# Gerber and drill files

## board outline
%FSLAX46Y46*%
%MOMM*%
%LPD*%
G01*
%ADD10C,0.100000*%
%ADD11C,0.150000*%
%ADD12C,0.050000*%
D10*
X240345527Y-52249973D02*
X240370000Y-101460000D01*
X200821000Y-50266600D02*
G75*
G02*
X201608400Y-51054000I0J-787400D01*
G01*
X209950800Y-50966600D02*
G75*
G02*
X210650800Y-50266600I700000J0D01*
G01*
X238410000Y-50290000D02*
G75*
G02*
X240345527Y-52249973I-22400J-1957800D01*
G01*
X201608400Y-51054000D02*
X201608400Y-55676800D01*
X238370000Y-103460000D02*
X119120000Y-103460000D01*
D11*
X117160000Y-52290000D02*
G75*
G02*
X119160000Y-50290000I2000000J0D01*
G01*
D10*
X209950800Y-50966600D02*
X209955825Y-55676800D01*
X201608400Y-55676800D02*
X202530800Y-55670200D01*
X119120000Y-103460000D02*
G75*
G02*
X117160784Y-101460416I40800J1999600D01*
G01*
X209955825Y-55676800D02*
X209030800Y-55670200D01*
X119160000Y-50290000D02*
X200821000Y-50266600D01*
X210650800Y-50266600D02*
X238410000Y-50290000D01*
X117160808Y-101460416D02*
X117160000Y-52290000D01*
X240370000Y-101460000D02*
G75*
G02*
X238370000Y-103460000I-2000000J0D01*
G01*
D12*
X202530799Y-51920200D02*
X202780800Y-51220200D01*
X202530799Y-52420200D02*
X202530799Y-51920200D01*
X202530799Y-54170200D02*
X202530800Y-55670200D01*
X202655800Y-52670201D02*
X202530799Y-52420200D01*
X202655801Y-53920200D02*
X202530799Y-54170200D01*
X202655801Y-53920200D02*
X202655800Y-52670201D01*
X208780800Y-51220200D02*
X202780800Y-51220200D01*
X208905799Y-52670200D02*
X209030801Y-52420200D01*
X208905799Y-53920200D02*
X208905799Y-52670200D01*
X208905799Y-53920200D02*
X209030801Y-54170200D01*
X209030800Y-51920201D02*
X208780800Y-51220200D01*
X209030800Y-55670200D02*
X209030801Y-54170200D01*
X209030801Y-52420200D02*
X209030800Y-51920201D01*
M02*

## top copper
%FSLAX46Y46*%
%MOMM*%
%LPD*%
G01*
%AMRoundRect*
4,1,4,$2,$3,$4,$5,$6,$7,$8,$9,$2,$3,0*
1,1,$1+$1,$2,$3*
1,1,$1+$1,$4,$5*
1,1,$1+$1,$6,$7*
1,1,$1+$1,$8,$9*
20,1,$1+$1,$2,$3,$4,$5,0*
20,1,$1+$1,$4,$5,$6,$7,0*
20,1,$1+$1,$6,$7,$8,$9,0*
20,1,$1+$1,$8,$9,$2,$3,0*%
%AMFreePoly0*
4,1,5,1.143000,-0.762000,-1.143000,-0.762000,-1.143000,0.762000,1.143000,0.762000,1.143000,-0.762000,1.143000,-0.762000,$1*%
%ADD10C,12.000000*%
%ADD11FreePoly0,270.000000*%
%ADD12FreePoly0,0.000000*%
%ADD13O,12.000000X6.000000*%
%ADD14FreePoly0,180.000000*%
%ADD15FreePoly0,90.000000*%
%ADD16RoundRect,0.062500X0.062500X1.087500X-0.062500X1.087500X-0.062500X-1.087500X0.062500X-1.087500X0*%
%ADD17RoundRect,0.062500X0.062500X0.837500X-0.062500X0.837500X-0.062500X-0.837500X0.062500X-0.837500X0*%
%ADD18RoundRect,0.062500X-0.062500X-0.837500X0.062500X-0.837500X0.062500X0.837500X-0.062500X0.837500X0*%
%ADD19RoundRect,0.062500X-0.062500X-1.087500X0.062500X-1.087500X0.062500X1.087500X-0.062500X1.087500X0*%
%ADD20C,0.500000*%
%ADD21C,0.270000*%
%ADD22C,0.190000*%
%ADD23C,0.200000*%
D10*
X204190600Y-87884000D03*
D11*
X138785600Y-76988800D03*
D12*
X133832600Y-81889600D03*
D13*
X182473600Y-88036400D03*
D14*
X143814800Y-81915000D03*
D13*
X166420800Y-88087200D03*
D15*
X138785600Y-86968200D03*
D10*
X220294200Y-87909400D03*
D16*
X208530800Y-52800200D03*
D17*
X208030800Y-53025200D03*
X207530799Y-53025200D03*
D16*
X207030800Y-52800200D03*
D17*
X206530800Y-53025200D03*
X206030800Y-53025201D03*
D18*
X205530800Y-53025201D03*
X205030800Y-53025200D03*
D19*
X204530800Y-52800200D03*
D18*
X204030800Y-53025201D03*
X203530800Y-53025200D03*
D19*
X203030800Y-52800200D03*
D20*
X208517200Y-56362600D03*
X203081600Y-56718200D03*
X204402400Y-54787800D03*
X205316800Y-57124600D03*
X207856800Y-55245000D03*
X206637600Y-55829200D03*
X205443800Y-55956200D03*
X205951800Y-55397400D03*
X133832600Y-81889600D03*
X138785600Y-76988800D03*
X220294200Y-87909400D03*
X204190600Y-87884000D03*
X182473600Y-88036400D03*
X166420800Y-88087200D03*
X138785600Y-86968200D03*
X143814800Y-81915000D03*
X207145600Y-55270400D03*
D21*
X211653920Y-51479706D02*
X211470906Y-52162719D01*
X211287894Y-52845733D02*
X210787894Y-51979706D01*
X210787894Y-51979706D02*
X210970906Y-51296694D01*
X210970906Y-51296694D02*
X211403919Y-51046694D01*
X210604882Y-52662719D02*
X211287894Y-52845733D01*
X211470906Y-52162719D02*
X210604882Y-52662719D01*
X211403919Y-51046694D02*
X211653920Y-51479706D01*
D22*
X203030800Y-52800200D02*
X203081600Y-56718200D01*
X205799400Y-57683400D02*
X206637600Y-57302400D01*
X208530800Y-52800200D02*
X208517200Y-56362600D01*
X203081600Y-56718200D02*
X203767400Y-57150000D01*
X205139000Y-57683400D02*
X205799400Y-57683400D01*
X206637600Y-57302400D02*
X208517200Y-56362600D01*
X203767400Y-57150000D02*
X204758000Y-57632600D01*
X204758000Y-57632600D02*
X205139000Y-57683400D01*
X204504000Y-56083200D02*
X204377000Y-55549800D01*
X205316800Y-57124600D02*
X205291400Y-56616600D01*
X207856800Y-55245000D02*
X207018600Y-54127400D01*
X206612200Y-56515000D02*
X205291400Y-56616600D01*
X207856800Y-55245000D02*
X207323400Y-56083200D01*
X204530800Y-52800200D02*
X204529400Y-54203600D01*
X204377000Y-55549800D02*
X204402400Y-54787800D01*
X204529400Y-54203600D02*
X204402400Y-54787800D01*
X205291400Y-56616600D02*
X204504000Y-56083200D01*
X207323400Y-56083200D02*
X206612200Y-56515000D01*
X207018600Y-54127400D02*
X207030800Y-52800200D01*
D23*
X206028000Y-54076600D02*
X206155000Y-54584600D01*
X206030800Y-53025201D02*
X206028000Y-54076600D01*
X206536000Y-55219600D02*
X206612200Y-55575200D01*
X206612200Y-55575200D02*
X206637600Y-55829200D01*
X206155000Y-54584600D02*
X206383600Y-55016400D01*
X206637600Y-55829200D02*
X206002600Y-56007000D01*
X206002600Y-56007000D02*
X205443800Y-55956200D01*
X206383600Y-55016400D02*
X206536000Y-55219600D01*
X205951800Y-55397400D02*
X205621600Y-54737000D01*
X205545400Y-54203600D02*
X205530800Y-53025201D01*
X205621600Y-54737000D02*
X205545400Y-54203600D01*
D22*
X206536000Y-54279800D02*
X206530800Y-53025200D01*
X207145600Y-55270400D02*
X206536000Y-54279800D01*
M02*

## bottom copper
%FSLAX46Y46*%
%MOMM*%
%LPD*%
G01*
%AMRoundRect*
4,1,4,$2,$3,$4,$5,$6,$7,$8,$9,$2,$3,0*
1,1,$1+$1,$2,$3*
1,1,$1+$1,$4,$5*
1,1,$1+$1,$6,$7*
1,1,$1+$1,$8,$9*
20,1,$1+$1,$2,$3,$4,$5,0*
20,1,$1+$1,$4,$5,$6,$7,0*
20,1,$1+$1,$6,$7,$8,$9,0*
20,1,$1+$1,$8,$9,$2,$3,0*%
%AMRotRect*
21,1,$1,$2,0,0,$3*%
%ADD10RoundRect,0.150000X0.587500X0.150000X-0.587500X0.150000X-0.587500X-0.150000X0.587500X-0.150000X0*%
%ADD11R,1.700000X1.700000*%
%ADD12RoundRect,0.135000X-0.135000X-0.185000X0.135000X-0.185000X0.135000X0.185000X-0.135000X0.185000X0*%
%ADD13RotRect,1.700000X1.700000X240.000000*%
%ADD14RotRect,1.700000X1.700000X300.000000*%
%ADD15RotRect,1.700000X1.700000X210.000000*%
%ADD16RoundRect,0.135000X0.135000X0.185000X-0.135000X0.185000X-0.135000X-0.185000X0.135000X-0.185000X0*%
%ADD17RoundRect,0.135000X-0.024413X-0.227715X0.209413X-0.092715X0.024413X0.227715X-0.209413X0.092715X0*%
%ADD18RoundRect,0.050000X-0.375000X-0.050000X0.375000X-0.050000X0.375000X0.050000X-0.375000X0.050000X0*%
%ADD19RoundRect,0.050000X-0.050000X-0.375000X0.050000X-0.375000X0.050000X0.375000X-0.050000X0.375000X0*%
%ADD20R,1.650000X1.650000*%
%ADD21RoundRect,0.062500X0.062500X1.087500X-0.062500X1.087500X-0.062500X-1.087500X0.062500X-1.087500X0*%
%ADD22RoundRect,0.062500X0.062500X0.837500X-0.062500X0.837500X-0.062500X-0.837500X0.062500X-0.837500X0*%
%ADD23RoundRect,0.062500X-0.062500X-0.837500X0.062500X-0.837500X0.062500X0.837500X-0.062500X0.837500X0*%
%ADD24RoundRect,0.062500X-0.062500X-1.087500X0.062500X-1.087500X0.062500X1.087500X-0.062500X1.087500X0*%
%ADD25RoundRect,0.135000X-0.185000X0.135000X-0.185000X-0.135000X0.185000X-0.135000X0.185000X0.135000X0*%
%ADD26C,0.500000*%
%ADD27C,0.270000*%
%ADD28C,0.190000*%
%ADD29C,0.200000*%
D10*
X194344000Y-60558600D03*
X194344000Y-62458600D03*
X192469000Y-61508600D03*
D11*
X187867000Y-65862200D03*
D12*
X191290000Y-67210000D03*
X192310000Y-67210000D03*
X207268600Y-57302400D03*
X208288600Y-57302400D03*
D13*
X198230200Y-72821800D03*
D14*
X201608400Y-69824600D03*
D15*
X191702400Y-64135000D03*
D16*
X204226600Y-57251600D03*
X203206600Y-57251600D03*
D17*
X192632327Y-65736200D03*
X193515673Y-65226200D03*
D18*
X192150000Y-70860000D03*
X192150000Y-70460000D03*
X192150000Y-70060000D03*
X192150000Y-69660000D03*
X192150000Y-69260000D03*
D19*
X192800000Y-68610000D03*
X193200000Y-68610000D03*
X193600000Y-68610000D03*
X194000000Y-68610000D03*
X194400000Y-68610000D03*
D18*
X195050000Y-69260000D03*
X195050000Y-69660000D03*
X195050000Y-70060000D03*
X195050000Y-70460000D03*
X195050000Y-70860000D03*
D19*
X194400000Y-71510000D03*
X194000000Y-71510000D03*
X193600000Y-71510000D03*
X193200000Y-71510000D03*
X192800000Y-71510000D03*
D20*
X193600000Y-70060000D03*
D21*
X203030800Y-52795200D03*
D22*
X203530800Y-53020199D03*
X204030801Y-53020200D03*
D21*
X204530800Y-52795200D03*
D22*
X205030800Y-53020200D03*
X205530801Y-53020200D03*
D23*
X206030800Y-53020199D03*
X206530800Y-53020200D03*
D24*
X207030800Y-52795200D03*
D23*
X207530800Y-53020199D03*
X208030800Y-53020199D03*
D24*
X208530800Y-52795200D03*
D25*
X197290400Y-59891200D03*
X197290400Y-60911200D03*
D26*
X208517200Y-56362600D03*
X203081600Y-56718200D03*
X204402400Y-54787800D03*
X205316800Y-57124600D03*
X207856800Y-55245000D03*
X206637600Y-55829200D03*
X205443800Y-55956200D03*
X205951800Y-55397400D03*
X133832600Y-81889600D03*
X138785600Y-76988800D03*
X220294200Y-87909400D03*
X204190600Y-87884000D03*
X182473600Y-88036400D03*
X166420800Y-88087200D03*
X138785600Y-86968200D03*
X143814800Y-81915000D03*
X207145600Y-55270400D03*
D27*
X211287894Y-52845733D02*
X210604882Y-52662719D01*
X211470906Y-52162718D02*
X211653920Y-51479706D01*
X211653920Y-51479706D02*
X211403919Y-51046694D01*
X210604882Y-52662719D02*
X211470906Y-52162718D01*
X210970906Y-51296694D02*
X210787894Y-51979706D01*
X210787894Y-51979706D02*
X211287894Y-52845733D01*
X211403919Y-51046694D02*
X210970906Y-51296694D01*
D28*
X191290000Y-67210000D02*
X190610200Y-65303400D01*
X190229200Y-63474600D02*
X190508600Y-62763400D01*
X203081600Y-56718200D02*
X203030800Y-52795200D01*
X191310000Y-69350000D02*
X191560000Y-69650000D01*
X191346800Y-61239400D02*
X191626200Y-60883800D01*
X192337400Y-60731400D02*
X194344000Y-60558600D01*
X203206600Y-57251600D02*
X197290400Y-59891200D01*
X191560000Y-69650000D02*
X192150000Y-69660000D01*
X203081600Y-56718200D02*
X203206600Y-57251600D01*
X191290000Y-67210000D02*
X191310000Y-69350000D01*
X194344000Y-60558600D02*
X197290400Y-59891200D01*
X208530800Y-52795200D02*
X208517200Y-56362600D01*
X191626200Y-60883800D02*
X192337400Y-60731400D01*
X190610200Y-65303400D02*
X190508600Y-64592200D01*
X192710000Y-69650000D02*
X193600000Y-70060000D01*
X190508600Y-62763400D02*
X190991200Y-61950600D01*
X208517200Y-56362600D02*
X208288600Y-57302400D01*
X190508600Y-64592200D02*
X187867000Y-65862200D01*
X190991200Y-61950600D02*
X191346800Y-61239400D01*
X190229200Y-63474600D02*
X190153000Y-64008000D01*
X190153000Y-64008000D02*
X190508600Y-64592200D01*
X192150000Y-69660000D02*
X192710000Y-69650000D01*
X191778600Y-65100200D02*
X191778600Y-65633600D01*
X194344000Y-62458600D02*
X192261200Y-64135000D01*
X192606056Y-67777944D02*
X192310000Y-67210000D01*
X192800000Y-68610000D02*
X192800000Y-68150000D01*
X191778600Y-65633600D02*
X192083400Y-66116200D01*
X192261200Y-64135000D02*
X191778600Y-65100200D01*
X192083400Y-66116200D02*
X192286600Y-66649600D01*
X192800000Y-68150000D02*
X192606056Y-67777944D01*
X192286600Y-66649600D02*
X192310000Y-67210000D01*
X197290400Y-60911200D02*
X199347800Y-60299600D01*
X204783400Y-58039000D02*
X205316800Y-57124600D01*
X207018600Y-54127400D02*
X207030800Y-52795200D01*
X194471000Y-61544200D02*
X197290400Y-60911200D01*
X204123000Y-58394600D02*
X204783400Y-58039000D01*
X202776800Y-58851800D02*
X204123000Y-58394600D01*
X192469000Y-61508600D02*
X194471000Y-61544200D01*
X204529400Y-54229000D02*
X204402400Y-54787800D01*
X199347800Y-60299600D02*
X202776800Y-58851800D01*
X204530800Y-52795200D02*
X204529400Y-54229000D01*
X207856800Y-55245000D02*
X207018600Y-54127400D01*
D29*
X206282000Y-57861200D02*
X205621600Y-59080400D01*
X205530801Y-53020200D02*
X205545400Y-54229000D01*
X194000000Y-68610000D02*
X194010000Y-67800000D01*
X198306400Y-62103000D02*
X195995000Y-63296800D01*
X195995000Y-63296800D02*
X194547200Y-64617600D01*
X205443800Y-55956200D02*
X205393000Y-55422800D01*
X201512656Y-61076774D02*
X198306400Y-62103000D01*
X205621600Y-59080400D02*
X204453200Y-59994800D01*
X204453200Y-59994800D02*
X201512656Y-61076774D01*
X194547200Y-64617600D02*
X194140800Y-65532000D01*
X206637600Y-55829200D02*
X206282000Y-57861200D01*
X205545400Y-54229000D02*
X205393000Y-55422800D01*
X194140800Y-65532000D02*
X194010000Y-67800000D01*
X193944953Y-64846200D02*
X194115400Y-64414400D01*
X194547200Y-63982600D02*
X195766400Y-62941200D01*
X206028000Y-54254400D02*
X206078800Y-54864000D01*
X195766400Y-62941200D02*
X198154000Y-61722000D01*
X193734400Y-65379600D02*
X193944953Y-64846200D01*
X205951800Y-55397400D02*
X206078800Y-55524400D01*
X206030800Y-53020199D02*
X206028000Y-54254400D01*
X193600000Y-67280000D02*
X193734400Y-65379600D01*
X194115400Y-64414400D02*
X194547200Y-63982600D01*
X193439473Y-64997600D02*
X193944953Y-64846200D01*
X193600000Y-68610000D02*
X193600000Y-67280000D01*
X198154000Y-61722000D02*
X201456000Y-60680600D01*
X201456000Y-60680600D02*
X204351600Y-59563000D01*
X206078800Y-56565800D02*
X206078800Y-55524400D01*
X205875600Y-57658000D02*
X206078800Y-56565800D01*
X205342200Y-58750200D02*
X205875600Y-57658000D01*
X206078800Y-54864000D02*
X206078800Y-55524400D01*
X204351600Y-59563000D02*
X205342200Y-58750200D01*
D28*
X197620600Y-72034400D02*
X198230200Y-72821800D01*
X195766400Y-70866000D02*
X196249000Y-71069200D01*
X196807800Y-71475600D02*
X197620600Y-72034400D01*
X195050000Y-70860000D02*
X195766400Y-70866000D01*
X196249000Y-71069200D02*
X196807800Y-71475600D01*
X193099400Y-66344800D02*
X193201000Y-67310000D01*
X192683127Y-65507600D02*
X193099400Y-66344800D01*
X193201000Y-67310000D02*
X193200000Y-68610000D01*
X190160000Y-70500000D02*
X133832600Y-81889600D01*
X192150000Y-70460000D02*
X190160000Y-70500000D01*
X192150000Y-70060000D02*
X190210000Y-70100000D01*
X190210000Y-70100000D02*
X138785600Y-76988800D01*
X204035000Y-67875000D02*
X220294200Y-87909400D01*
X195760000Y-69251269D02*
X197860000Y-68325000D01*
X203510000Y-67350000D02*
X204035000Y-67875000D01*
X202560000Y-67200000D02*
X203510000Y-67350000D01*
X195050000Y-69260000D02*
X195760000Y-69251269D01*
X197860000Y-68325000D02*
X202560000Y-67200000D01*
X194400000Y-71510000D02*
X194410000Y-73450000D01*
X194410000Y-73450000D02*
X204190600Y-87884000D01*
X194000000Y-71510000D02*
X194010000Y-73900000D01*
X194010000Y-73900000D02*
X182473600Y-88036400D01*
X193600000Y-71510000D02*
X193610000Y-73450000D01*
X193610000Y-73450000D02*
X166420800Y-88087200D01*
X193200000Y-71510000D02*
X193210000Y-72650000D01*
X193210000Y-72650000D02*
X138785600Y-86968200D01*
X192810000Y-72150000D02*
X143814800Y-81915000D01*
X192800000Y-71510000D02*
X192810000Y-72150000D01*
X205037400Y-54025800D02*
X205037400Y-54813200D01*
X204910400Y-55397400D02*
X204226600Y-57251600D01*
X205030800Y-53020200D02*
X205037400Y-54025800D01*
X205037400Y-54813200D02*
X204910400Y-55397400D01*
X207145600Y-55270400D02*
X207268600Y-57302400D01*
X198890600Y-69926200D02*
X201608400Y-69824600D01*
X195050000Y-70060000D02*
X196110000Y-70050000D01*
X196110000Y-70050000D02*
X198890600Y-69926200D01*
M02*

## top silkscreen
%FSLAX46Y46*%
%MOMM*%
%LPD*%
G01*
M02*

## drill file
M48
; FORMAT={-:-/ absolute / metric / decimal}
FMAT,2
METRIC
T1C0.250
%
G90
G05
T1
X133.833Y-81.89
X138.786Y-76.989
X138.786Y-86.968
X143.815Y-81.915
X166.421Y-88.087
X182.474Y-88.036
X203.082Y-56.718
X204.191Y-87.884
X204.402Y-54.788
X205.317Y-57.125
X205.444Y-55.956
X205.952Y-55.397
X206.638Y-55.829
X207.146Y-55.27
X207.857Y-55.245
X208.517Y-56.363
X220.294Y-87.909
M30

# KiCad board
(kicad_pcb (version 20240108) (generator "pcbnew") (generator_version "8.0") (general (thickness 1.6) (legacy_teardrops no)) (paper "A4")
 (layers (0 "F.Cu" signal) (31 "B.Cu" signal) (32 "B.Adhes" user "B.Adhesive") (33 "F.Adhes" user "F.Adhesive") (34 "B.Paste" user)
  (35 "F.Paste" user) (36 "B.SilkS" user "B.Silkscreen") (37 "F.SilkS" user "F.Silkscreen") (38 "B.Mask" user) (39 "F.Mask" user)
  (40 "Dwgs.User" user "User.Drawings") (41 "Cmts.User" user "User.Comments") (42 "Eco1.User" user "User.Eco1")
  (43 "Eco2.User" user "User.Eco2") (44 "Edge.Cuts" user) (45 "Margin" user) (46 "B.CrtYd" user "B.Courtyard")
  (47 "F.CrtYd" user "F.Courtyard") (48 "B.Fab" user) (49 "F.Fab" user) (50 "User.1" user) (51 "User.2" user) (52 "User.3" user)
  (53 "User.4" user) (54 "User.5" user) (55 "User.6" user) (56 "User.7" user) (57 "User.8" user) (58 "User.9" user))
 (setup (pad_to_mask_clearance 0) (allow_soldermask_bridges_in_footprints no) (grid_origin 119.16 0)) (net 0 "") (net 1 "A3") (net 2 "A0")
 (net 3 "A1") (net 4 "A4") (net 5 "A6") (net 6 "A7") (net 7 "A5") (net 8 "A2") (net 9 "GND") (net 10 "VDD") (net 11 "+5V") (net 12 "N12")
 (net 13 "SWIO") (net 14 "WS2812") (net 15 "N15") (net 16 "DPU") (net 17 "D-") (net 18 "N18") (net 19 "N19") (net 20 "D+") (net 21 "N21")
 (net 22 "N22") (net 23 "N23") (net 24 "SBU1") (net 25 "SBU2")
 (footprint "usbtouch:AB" (layer "F.Cu") (at 204.1906 87.884)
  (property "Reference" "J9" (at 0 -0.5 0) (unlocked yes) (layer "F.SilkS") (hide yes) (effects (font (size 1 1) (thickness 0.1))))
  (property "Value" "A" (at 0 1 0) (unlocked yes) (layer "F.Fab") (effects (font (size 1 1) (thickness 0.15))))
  (pad "1" smd circle (at 0 0) (size 12 12) (layers "F.Cu") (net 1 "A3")))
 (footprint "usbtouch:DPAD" (layer "F.Cu") (at 138.7856 76.9888 -90)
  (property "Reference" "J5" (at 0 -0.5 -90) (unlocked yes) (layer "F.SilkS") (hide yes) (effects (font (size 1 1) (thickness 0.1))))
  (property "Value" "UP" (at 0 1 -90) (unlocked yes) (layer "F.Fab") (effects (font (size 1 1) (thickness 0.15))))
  (pad "1" smd custom (at 0 0 270) (size 2.286 1.524) (layers "F.Cu") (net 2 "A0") (thermal_bridge_angle 45)
   (options (clearance outline) (anchor rect)) (primitives)))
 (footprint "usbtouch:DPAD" (layer "F.Cu") (at 133.8326 81.8896)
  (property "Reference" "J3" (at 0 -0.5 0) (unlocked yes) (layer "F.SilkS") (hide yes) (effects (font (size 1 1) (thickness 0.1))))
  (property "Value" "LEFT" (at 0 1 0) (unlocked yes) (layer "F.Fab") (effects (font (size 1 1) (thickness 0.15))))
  (pad "1" smd custom (at 0 0) (size 2.286 1.524) (layers "F.Cu") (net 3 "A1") (thermal_bridge_angle 45)
   (options (clearance outline) (anchor rect)) (primitives)))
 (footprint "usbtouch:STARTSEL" (layer "F.Cu") (at 182.4736 88.0364)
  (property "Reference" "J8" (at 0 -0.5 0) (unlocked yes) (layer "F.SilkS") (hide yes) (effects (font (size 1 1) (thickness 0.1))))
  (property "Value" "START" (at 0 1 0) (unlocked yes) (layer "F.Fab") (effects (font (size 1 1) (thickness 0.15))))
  (pad "1" smd oval (at 0 0) (size 12 6) (layers "F.Cu") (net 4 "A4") (thermal_bridge_angle 45)))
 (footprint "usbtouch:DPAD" (layer "F.Cu") (at 143.8148 81.915 180)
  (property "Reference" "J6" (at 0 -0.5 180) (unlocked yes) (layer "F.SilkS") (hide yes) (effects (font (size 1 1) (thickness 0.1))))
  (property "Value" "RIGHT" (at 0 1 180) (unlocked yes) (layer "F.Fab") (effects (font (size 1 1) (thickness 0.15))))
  (pad "1" smd custom (at 0 0 180) (size 2.286 1.524) (layers "F.Cu") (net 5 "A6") (thermal_bridge_angle 45)
   (options (clearance outline) (anchor rect)) (primitives)))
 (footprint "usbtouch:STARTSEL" (layer "F.Cu") (at 166.4208 88.0872)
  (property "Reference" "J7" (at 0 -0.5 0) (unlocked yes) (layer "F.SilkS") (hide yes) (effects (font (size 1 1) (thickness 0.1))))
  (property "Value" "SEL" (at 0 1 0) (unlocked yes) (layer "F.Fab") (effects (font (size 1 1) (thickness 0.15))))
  (pad "1" smd oval (at 0 0) (size 12 6) (layers "F.Cu") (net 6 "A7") (thermal_bridge_angle 45)))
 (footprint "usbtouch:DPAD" (layer "F.Cu") (at 138.7856 86.9682 90)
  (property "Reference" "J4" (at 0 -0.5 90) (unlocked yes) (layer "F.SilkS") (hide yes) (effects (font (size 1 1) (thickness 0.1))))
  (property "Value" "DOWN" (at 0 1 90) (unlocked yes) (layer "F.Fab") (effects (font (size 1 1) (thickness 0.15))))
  (pad "1" smd custom (at 0 0 90) (size 2.286 1.524) (layers "F.Cu") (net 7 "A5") (thermal_bridge_angle 45)
   (options (clearance outline) (anchor rect)) (primitives)))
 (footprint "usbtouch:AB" (layer "F.Cu") (at 220.2942 87.9094)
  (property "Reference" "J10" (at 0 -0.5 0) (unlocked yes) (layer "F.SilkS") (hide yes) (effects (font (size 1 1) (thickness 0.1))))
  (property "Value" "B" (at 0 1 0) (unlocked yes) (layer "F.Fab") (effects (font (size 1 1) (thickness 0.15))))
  (pad "1" smd circle (at 0 0) (size 12 12) (layers "F.Cu") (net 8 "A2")))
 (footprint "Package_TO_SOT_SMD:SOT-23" (layer "B.Cu") (at 193.4065 61.5086 180)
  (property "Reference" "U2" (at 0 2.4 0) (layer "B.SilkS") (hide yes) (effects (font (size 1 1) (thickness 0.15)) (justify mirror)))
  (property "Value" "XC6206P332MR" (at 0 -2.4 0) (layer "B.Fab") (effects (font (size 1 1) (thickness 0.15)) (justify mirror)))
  (pad "1" smd roundrect (at -0.9375 0.95 180) (size 1.475 0.6) (layers "B.Cu" "B.Paste" "B.Mask") (roundrect_rratio 0.25) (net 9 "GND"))
  (pad "2" smd roundrect (at -0.9375 -0.95 180) (size 1.475 0.6) (layers "B.Cu" "B.Paste" "B.Mask") (roundrect_rratio 0.25) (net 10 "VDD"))
  (pad "3" smd roundrect (at 0.9375 0 180) (size 1.475 0.6) (layers "B.Cu" "B.Paste" "B.Mask") (roundrect_rratio 0.25) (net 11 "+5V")))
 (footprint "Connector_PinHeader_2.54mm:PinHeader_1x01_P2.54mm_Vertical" (layer "B.Cu") (at 187.867 65.8622 -90)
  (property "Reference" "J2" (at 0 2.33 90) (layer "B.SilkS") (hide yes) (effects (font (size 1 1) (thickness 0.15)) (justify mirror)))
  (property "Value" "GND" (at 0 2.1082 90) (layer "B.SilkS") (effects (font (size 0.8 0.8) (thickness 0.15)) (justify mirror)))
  (pad "1" smd rect (at 0 0 270) (size 1.7 1.7) (layers "B.Cu" "B.Paste" "B.Mask") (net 9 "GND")))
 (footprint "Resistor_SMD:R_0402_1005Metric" (layer "B.Cu") (at 191.8 67.21)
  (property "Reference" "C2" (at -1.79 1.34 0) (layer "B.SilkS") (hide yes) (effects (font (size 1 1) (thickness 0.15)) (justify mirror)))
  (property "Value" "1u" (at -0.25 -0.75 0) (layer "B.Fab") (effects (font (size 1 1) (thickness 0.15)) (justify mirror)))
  (pad "1" smd roundrect (at -0.51 0) (size 0.54 0.64) (layers "B.Cu" "B.Paste" "B.Mask") (roundrect_rratio 0.25) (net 9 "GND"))
  (pad "2" smd roundrect (at 0.51 0) (size 0.54 0.64) (layers "B.Cu" "B.Paste" "B.Mask") (roundrect_rratio 0.25) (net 10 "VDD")))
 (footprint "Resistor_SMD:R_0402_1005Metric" (layer "B.Cu") (at 207.7786 57.3024)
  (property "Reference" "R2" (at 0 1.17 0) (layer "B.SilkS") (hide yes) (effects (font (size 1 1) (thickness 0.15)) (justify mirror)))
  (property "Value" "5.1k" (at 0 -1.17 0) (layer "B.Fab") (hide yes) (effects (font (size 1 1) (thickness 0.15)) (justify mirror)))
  (pad "1" smd roundrect (at -0.51 0) (size 0.54 0.64) (layers "B.Cu" "B.Paste" "B.Mask") (roundrect_rratio 0.25) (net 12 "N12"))
  (pad "2" smd roundrect (at 0.51 0) (size 0.54 0.64) (layers "B.Cu" "B.Paste" "B.Mask") (roundrect_rratio 0.25) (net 9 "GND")))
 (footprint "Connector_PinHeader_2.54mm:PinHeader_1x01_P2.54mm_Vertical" (layer "B.Cu") (at 198.2302 72.8218 -120)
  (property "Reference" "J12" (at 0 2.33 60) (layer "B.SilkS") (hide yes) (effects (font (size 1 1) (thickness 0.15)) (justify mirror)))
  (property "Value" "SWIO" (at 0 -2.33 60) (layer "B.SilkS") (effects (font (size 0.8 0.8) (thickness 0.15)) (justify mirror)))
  (pad "1" smd rect (at 0 0 240) (size 1.7 1.7) (layers "B.Cu" "B.Paste" "B.Mask") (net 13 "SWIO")))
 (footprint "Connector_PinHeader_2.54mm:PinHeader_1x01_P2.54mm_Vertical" (layer "B.Cu") (at 201.6084 69.8246 -60)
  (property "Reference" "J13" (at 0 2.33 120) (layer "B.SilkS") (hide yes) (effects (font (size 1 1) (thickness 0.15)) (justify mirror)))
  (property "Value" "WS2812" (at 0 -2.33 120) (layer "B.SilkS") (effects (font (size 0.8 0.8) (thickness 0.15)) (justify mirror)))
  (pad "1" smd rect (at 0 0 300) (size 1.7 1.7) (layers "B.Cu" "B.Paste" "B.Mask") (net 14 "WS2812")))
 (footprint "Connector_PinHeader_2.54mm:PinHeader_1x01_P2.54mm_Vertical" (layer "B.Cu") (at 191.7024 64.135 -150)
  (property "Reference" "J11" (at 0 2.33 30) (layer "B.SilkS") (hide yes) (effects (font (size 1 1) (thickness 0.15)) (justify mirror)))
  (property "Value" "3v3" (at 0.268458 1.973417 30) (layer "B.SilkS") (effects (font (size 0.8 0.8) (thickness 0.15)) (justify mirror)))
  (pad "1" smd rect (at 0 0 210) (size 1.7 1.7) (layers "B.Cu" "B.Paste" "B.Mask") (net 10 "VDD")))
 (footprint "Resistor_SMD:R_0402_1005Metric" (layer "B.Cu") (at 203.7166 57.2516 180)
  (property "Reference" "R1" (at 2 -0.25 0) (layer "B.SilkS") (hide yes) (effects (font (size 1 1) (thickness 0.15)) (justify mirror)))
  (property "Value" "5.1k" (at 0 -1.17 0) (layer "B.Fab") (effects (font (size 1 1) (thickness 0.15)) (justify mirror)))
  (pad "1" smd roundrect (at -0.51 0 180) (size 0.54 0.64) (layers "B.Cu" "B.Paste" "B.Mask") (roundrect_rratio 0.25) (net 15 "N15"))
  (pad "2" smd roundrect (at 0.51 0 180) (size 0.54 0.64) (layers "B.Cu" "B.Paste" "B.Mask") (roundrect_rratio 0.25) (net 9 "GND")))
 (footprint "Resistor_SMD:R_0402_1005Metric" (layer "B.Cu") (at 193.074 65.4812 30)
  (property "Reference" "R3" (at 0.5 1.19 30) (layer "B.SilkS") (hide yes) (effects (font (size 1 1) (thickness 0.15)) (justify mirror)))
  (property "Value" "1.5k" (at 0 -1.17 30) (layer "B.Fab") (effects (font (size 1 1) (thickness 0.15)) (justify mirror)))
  (pad "1" smd roundrect (at -0.51 0 30) (size 0.54 0.64) (layers "B.Cu" "B.Paste" "B.Mask") (roundrect_rratio 0.25) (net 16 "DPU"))
  (pad "2" smd roundrect (at 0.51 0 30) (size 0.54 0.64) (layers "B.Cu" "B.Paste" "B.Mask") (roundrect_rratio 0.25) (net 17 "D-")))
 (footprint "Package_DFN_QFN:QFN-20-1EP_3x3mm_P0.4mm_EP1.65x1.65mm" (layer "B.Cu") (at 193.6 70.06)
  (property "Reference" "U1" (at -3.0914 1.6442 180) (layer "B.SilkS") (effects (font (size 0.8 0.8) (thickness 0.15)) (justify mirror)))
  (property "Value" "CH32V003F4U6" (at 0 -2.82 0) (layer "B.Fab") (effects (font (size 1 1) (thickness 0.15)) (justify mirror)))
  (pad "" smd roundrect (at -0.41 -0.41) (size 0.67 0.67) (layers "B.Paste") (roundrect_rratio 0.25))
  (pad "" smd roundrect (at -0.41 0.41) (size 0.67 0.67) (layers "B.Paste") (roundrect_rratio 0.25))
  (pad "" smd roundrect (at 0.41 -0.41) (size 0.67 0.67) (layers "B.Paste") (roundrect_rratio 0.25))
  (pad "" smd roundrect (at 0.41 0.41) (size 0.67 0.67) (layers "B.Paste") (roundrect_rratio 0.25))
  (pad "1" smd roundrect (at -1.45 0.8) (size 0.85 0.2) (layers "B.Cu" "B.Paste" "B.Mask") (roundrect_rratio 0.25) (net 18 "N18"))
  (pad "2" smd roundrect (at -1.45 0.4) (size 0.85 0.2) (layers "B.Cu" "B.Paste" "B.Mask") (roundrect_rratio 0.25) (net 3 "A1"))
  (pad "3" smd roundrect (at -1.45 0) (size 0.85 0.2) (layers "B.Cu" "B.Paste" "B.Mask") (roundrect_rratio 0.25) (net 2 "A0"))
  (pad "4" smd roundrect (at -1.45 -0.4) (size 0.85 0.2) (layers "B.Cu" "B.Paste" "B.Mask") (roundrect_rratio 0.25) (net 9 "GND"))
  (pad "5" smd roundrect (at -1.45 -0.8) (size 0.85 0.2) (layers "B.Cu" "B.Paste" "B.Mask") (roundrect_rratio 0.25) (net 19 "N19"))
  (pad "6" smd roundrect (at -0.8 -1.45) (size 0.2 0.85) (layers "B.Cu" "B.Paste" "B.Mask") (roundrect_rratio 0.25) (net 10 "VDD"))
  (pad "7" smd roundrect (at -0.4 -1.45) (size 0.2 0.85) (layers "B.Cu" "B.Paste" "B.Mask") (roundrect_rratio 0.25) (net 16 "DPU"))
  (pad "8" smd roundrect (at 0 -1.45) (size 0.2 0.85) (layers "B.Cu" "B.Paste" "B.Mask") (roundrect_rratio 0.25) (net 17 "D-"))
  (pad "9" smd roundrect (at 0.4 -1.45) (size 0.2 0.85) (layers "B.Cu" "B.Paste" "B.Mask") (roundrect_rratio 0.25) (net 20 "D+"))
  (pad "10" smd roundrect (at 0.8 -1.45) (size 0.2 0.85) (layers "B.Cu" "B.Paste" "B.Mask") (roundrect_rratio 0.25) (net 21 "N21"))
  (pad "11" smd roundrect (at 1.45 -0.8) (size 0.85 0.2) (layers "B.Cu" "B.Paste" "B.Mask") (roundrect_rratio 0.25) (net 8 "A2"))
  (pad "12" smd roundrect (at 1.45 -0.4) (size 0.85 0.2) (layers "B.Cu" "B.Paste" "B.Mask") (roundrect_rratio 0.25) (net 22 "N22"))
  (pad "13" smd roundrect (at 1.45 0) (size 0.85 0.2) (layers "B.Cu" "B.Paste" "B.Mask") (roundrect_rratio 0.25) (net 14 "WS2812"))
  (pad "14" smd roundrect (at 1.45 0.4) (size 0.85 0.2) (layers "B.Cu" "B.Paste" "B.Mask") (roundrect_rratio 0.25) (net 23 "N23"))
  (pad "15" smd roundrect (at 1.45 0.8) (size 0.85 0.2) (layers "B.Cu" "B.Paste" "B.Mask") (roundrect_rratio 0.25) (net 13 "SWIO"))
  (pad "16" smd roundrect (at 0.8 1.45) (size 0.2 0.85) (layers "B.Cu" "B.Paste" "B.Mask") (roundrect_rratio 0.25) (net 1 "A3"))
  (pad "17" smd roundrect (at 0.4 1.45) (size 0.2 0.85) (layers "B.Cu" "B.Paste" "B.Mask") (roundrect_rratio 0.25) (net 4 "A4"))
  (pad "18" smd roundrect (at 0 1.45) (size 0.2 0.85) (layers "B.Cu" "B.Paste" "B.Mask") (roundrect_rratio 0.25) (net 6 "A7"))
  (pad "19" smd roundrect (at -0.4 1.45) (size 0.2 0.85) (layers "B.Cu" "B.Paste" "B.Mask") (roundrect_rratio 0.25) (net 7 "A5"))
  (pad "20" smd roundrect (at -0.8 1.45) (size 0.2 0.85) (layers "B.Cu" "B.Paste" "B.Mask") (roundrect_rratio 0.25) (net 5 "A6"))
  (pad "21" smd rect (at 0 0) (size 1.65 1.65) (layers "B.Cu" "B.Mask") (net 9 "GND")))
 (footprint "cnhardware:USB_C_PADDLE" (layer "B.Cu") (at 205.7808 53.6702 180)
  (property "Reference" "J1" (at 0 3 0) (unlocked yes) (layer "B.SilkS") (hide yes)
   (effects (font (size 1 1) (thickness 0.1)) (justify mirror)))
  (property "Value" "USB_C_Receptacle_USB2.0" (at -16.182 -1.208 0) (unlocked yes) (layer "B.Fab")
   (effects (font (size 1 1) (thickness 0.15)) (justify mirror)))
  (fp_line (start 3.250001 1.75) (end 3 2.45) (stroke (width 0.05) (type default)) (layer "Edge.Cuts"))
  (fp_line (start 3.250001 1.25) (end 3.250001 1.75) (stroke (width 0.05) (type default)) (layer "Edge.Cuts"))
  (fp_line (start 3.250001 -0.5) (end 3.25 -2) (stroke (width 0.05) (type default)) (layer "Edge.Cuts"))
  (fp_line (start 3.125 0.999999) (end 3.250001 1.25) (stroke (width 0.05) (type default)) (layer "Edge.Cuts"))
  (fp_line (start 3.124999 -0.25) (end 3.250001 -0.5) (stroke (width 0.05) (type default)) (layer "Edge.Cuts"))
  (fp_line (start 3.124999 -0.25) (end 3.125 0.999999) (stroke (width 0.05) (type default)) (layer "Edge.Cuts"))
  (fp_line (start -3 2.45) (end 3 2.45) (stroke (width 0.05) (type default)) (layer "Edge.Cuts"))
  (fp_line (start -3.124999 1) (end -3.250001 1.25) (stroke (width 0.05) (type default)) (layer "Edge.Cuts"))
  (fp_line (start -3.124999 -0.25) (end -3.124999 1) (stroke (width 0.05) (type default)) (layer "Edge.Cuts"))
  (fp_line (start -3.124999 -0.25) (end -3.250001 -0.5) (stroke (width 0.05) (type default)) (layer "Edge.Cuts"))
  (fp_line (start -3.25 1.749999) (end -3 2.45) (stroke (width 0.05) (type default)) (layer "Edge.Cuts"))
  (fp_line (start -3.25 -2) (end -3.250001 -0.5) (stroke (width 0.05) (type default)) (layer "Edge.Cuts"))
  (fp_line (start -3.250001 1.25) (end -3.25 1.749999) (stroke (width 0.05) (type default)) (layer "Edge.Cuts"))
  (pad "A1" smd roundrect (at 2.75 0.875 180) (size 0.25 2.3) (layers "B.Cu" "B.Paste" "B.Mask") (roundrect_rratio 0.25) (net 9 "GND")
   (thermal_bridge_angle 45))
  (pad "A2" smd roundrect (at 2.25 0.650001 180) (size 0.25 1.8) (layers "B.Cu" "B.Paste" "B.Mask") (roundrect_rratio 0.25)
   (thermal_bridge_angle 45))
  (pad "A3" smd roundrect (at 1.749999 0.65 180) (size 0.25 1.8) (layers "B.Cu" "B.Paste" "B.Mask") (roundrect_rratio 0.25)
   (thermal_bridge_angle 45))
  (pad "A4" smd roundrect (at 1.25 0.875 180) (size 0.25 2.3) (layers "B.Cu" "B.Paste" "B.Mask") (roundrect_rratio 0.25) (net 11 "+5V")
   (thermal_bridge_angle 45))
  (pad "A5" smd roundrect (at 0.75 0.65 180) (size 0.25 1.8) (layers "B.Cu" "B.Paste" "B.Mask") (roundrect_rratio 0.25) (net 15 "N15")
   (thermal_bridge_angle 45))
  (pad "A6" smd roundrect (at 0.249999 0.65 180) (size 0.25 1.8) (layers "B.Cu" "B.Paste" "B.Mask") (roundrect_rratio 0.25) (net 20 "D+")
   (thermal_bridge_angle 45))
  (pad "A7" smd roundrect (at -0.25 0.650001) (size 0.25 1.8) (layers "B.Cu" "B.Paste" "B.Mask") (roundrect_rratio 0.25) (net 17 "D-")
   (thermal_bridge_angle 45))
  (pad "A8" smd roundrect (at -0.75 0.65) (size 0.25 1.8) (layers "B.Cu" "B.Paste" "B.Mask") (roundrect_rratio 0.25) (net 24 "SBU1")
   (thermal_bridge_angle 45))
  (pad "A9" smd roundrect (at -1.25 0.875) (size 0.25 2.3) (layers "B.Cu" "B.Paste" "B.Mask") (roundrect_rratio 0.25) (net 11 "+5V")
   (thermal_bridge_angle 45))
  (pad "A10" smd roundrect (at -1.75 0.650001) (size 0.25 1.8) (layers "B.Cu" "B.Paste" "B.Mask") (roundrect_rratio 0.25)
   (thermal_bridge_angle 45))
  (pad "A11" smd roundrect (at -2.25 0.650001) (size 0.25 1.8) (layers "B.Cu" "B.Paste" "B.Mask") (roundrect_rratio 0.25)
   (thermal_bridge_angle 45))
  (pad "A12" smd roundrect (at -2.75 0.875) (size 0.25 2.3) (layers "B.Cu" "B.Paste" "B.Mask") (roundrect_rratio 0.25) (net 9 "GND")
   (thermal_bridge_angle 45))
  (pad "B1" smd roundrect (at -2.75 0.87 180) (size 0.25 2.3) (layers "F.Cu" "F.Paste" "F.Mask") (roundrect_rratio 0.25) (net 9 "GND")
   (thermal_bridge_angle 45))
  (pad "B2" smd roundrect (at -2.25 0.645 180) (size 0.25 1.8) (layers "F.Cu" "F.Paste" "F.Mask") (roundrect_rratio 0.25)
   (thermal_bridge_angle 45))
  (pad "B3" smd roundrect (at -1.749999 0.645 180) (size 0.25 1.8) (layers "F.Cu" "F.Paste" "F.Mask") (roundrect_rratio 0.25)
   (thermal_bridge_angle 45))
  (pad "B4" smd roundrect (at -1.25 0.87 180) (size 0.25 2.3) (layers "F.Cu" "F.Paste" "F.Mask") (roundrect_rratio 0.25) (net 11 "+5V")
   (thermal_bridge_angle 45))
  (pad "B5" smd roundrect (at -0.75 0.645 180) (size 0.25 1.8) (layers "F.Cu" "F.Paste" "F.Mask") (roundrect_rratio 0.25) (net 12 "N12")
   (thermal_bridge_angle 45))
  (pad "B6" smd roundrect (at -0.25 0.644999 180) (size 0.25 1.8) (layers "F.Cu" "F.Paste" "F.Mask") (roundrect_rratio 0.25) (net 20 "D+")
   (thermal_bridge_angle 45))
  (pad "B7" smd roundrect (at 0.25 0.644999) (size 0.25 1.8) (layers "F.Cu" "F.Paste" "F.Mask") (roundrect_rratio 0.25) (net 17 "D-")
   (thermal_bridge_angle 45))
  (pad "B8" smd roundrect (at 0.75 0.645) (size 0.25 1.8) (layers "F.Cu" "F.Paste" "F.Mask") (roundrect_rratio 0.25) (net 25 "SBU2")
   (thermal_bridge_angle 45))
  (pad "B9" smd roundrect (at 1.25 0.87) (size 0.25 2.3) (layers "F.Cu" "F.Paste" "F.Mask") (roundrect_rratio 0.25) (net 11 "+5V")
   (thermal_bridge_angle 45))
  (pad "B10" smd roundrect (at 1.75 0.644999) (size 0.25 1.8) (layers "F.Cu" "F.Paste" "F.Mask") (roundrect_rratio 0.25)
   (thermal_bridge_angle 45))
  (pad "B11" smd roundrect (at 2.25 0.645) (size 0.25 1.8) (layers "F.Cu" "F.Paste" "F.Mask") (roundrect_rratio 0.25)
   (thermal_bridge_angle 45))
  (pad "B12" smd roundrect (at 2.75 0.87) (size 0.25 2.3) (layers "F.Cu" "F.Paste" "F.Mask") (roundrect_rratio 0.25) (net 9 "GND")
   (thermal_bridge_angle 45)))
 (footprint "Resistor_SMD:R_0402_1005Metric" (layer "B.Cu") (at 197.2904 60.4012 -90)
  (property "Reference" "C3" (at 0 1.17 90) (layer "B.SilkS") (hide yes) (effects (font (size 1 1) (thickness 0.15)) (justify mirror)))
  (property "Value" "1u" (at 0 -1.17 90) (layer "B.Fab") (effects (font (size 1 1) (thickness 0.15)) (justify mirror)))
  (pad "1" smd roundrect (at -0.51 0 270) (size 0.54 0.64) (layers "B.Cu" "B.Paste" "B.Mask") (roundrect_rratio 0.25) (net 9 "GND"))
  (pad "2" smd roundrect (at 0.51 0 270) (size 0.54 0.64) (layers "B.Cu" "B.Paste" "B.Mask") (roundrect_rratio 0.25) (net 11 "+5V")))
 (gr_line (start 240.345527 52.249973) (end 240.37 101.46) (stroke (width 0.1) (type default)) (layer "Edge.Cuts"))
 (gr_arc (start 200.821 50.2666) (mid 201.377776 50.497224) (end 201.6084 51.054) (stroke (width 0.1) (type default)) (layer "Edge.Cuts"))
 (gr_arc (start 209.9508 50.9666) (mid 210.155833 50.471633) (end 210.6508 50.2666) (stroke (width 0.1) (type default)) (layer "Edge.Cuts"))
 (gr_arc (start 238.41 50.29) (mid 239.780725 50.872051) (end 240.345527 52.249973) (stroke (width 0.1) (type default)) (layer "Edge.Cuts"))
 (gr_line (start 201.6084 51.054) (end 201.6084 55.6768) (stroke (width 0.1) (type default)) (layer "Edge.Cuts"))
 (gr_line (start 238.37 103.46) (end 119.12 103.46) (stroke (width 0.1) (type default)) (layer "Edge.Cuts"))
 (gr_arc (start 117.16 52.29) (mid 117.745786 50.875786) (end 119.16 50.29) (stroke (width 0.15) (type default)) (layer "Edge.Cuts"))
 (gr_line (start 209.9508 50.9666) (end 209.955825 55.6768) (stroke (width 0.1) (type default)) (layer "Edge.Cuts"))
 (gr_line (start 201.6084 55.6768) (end 202.5308 55.6702) (stroke (width 0.1) (type default)) (layer "Edge.Cuts"))
 (gr_arc (start 119.12 103.46) (mid 117.732239 102.860128) (end 117.160808 101.460416) (stroke (width 0.1) (type default))
  (layer "Edge.Cuts"))
 (gr_line (start 209.955825 55.6768) (end 209.0308 55.6702) (stroke (width 0.1) (type default)) (layer "Edge.Cuts"))
 (gr_line (start 119.16 50.29) (end 200.821 50.2666) (stroke (width 0.1) (type default)) (layer "Edge.Cuts"))
 (gr_line (start 210.6508 50.2666) (end 238.41 50.29) (stroke (width 0.1) (type default)) (layer "Edge.Cuts"))
 (gr_line (start 117.160808 101.460416) (end 117.16 52.29) (stroke (width 0.1) (type default)) (layer "Edge.Cuts"))
 (gr_arc (start 240.37 101.46) (mid 239.784214 102.874214) (end 238.37 103.46) (stroke (width 0.1) (type default)) (layer "Edge.Cuts"))
 (segment (start 211.65392 51.479706) (end 211.470906 52.162719) (width 0.27) (layer "F.Cu") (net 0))
 (segment (start 211.287894 52.845733) (end 210.787894 51.979706) (width 0.27) (layer "F.Cu") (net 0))
 (segment (start 210.787894 51.979706) (end 210.970906 51.296694) (width 0.27) (layer "F.Cu") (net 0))
 (segment (start 210.970906 51.296694) (end 211.403919 51.046694) (width 0.27) (layer "F.Cu") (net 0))
 (segment (start 210.604882 52.662719) (end 211.287894 52.845733) (width 0.27) (layer "F.Cu") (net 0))
 (segment (start 211.470906 52.162719) (end 210.604882 52.662719) (width 0.27) (layer "F.Cu") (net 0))
 (segment (start 211.403919 51.046694) (end 211.65392 51.479706) (width 0.27) (layer "F.Cu") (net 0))
 (segment (start 211.287894 52.845733) (end 210.604882 52.662719) (width 0.27) (layer "B.Cu") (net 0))
 (segment (start 211.470906 52.162718) (end 211.65392 51.479706) (width 0.27) (layer "B.Cu") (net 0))
 (segment (start 211.65392 51.479706) (end 211.403919 51.046694) (width 0.27) (layer "B.Cu") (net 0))
 (segment (start 210.604882 52.662719) (end 211.470906 52.162718) (width 0.27) (layer "B.Cu") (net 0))
 (segment (start 210.970906 51.296694) (end 210.787894 51.979706) (width 0.27) (layer "B.Cu") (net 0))
 (segment (start 210.787894 51.979706) (end 211.287894 52.845733) (width 0.27) (layer "B.Cu") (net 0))
 (segment (start 211.403919 51.046694) (end 210.970906 51.296694) (width 0.27) (layer "B.Cu") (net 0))
 (segment (start 203.0308 52.8002) (end 203.0816 56.7182) (width 0.19) (layer "F.Cu") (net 9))
 (segment (start 205.7994 57.6834) (end 206.6376 57.3024) (width 0.19) (layer "F.Cu") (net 9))
 (segment (start 208.5308 52.8002) (end 208.5172 56.3626) (width 0.19) (layer "F.Cu") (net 9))
 (segment (start 203.0816 56.7182) (end 203.7674 57.15) (width 0.19) (layer "F.Cu") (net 9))
 (segment (start 205.139 57.6834) (end 205.7994 57.6834) (width 0.19) (layer "F.Cu") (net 9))
 (segment (start 206.6376 57.3024) (end 208.5172 56.3626) (width 0.19) (layer "F.Cu") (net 9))
 (segment (start 203.7674 57.15) (end 204.758 57.6326) (width 0.19) (layer "F.Cu") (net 9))
 (segment (start 204.758 57.6326) (end 205.139 57.6834) (width 0.19) (layer "F.Cu") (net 9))
 (via (at 208.5172 56.3626) (size 0.5) (drill 0.25) (layers "F.Cu" "B.Cu") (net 9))
 (via (at 203.0816 56.7182) (size 0.5) (drill 0.25) (layers "F.Cu" "B.Cu") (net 9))
 (segment (start 191.29 67.21) (end 190.6102 65.3034) (width 0.19) (layer "B.Cu") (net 9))
 (segment (start 190.2292 63.4746) (end 190.5086 62.7634) (width 0.19) (layer "B.Cu") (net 9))
 (segment (start 203.0816 56.7182) (end 203.0308 52.7952) (width 0.19) (layer "B.Cu") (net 9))
 (segment (start 191.31 69.35) (end 191.56 69.65) (width 0.19) (layer "B.Cu") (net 9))
 (segment (start 191.3468 61.2394) (end 191.6262 60.8838) (width 0.19) (layer "B.Cu") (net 9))
 (segment (start 192.3374 60.7314) (end 194.344 60.5586) (width 0.19) (layer "B.Cu") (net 9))
 (segment (start 203.2066 57.2516) (end 197.2904 59.8912) (width 0.19) (layer "B.Cu") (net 9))
 (segment (start 191.56 69.65) (end 192.15 69.66) (width 0.19) (layer "B.Cu") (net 9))
 (segment (start 203.0816 56.7182) (end 203.2066 57.2516) (width 0.19) (layer "B.Cu") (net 9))
 (segment (start 191.29 67.21) (end 191.31 69.35) (width 0.19) (layer "B.Cu") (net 9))
 (segment (start 194.344 60.5586) (end 197.2904 59.8912) (width 0.19) (layer "B.Cu") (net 9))
 (segment (start 208.5308 52.7952) (end 208.5172 56.3626) (width 0.19) (layer "B.Cu") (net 9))
 (segment (start 191.6262 60.8838) (end 192.3374 60.7314) (width 0.19) (layer "B.Cu") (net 9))
 (segment (start 190.6102 65.3034) (end 190.5086 64.5922) (width 0.19) (layer "B.Cu") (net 9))
 (segment (start 192.71 69.65) (end 193.6 70.06) (width 0.19) (layer "B.Cu") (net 9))
 (segment (start 190.5086 62.7634) (end 190.9912 61.9506) (width 0.19) (layer "B.Cu") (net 9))
 (segment (start 208.5172 56.3626) (end 208.2886 57.3024) (width 0.19) (layer "B.Cu") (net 9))
 (segment (start 190.5086 64.5922) (end 187.867 65.8622) (width 0.19) (layer "B.Cu") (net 9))
 (segment (start 190.9912 61.9506) (end 191.3468 61.2394) (width 0.19) (layer "B.Cu") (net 9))
 (segment (start 190.2292 63.4746) (end 190.153 64.008) (width 0.19) (layer "B.Cu") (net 9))
 (segment (start 190.153 64.008) (end 190.5086 64.5922) (width 0.19) (layer "B.Cu") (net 9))
 (segment (start 192.15 69.66) (end 192.71 69.65) (width 0.19) (layer "B.Cu") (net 9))
 (segment (start 191.7786 65.1002) (end 191.7786 65.6336) (width 0.19) (layer "B.Cu") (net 10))
 (segment (start 194.344 62.4586) (end 192.2612 64.135) (width 0.19) (layer "B.Cu") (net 10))
 (segment (start 192.606056 67.777944) (end 192.31 67.21) (width 0.19) (layer "B.Cu") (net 10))
 (segment (start 192.8 68.61) (end 192.8 68.15) (width 0.19) (layer "B.Cu") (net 10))
 (segment (start 191.7786 65.6336) (end 192.0834 66.1162) (width 0.19) (layer "B.Cu") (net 10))
 (segment (start 192.2612 64.135) (end 191.7786 65.1002) (width 0.19) (layer "B.Cu") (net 10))
 (segment (start 192.0834 66.1162) (end 192.2866 66.6496) (width 0.19) (layer "B.Cu") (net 10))
 (segment (start 192.8 68.15) (end 192.606056 67.777944) (width 0.19) (layer "B.Cu") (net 10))
 (segment (start 192.2866 66.6496) (end 192.31 67.21) (width 0.19) (layer "B.Cu") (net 10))
 (segment (start 204.504 56.0832) (end 204.377 55.5498) (width 0.19) (layer "F.Cu") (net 11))
 (segment (start 205.3168 57.1246) (end 205.2914 56.6166) (width 0.19) (layer "F.Cu") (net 11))
 (segment (start 207.8568 55.245) (end 207.0186 54.1274) (width 0.19) (layer "F.Cu") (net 11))
 (segment (start 206.6122 56.515) (end 205.2914 56.6166) (width 0.19) (layer "F.Cu") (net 11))
 (segment (start 207.8568 55.245) (end 207.3234 56.0832) (width 0.19) (layer "F.Cu") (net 11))
 (segment (start 204.5308 52.8002) (end 204.5294 54.2036) (width 0.19) (layer "F.Cu") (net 11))
 (segment (start 204.377 55.5498) (end 204.4024 54.7878) (width 0.19) (layer "F.Cu") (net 11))
 (segment (start 204.5294 54.2036) (end 204.4024 54.7878) (width 0.19) (layer "F.Cu") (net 11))
 (segment (start 205.2914 56.6166) (end 204.504 56.0832) (width 0.19) (layer "F.Cu") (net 11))
 (segment (start 207.3234 56.0832) (end 206.6122 56.515) (width 0.19) (layer "F.Cu") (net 11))
 (segment (start 207.0186 54.1274) (end 207.0308 52.8002) (width 0.19) (layer "F.Cu") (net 11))
 (via (at 204.4024 54.7878) (size 0.5) (drill 0.25) (layers "F.Cu" "B.Cu") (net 11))
 (via (at 205.3168 57.1246) (size 0.5) (drill 0.25) (layers "F.Cu" "B.Cu") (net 11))
 (via (at 207.8568 55.245) (size 0.5) (drill 0.25) (layers "F.Cu" "B.Cu") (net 11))
 (segment (start 197.2904 60.9112) (end 199.3478 60.2996) (width 0.19) (layer "B.Cu") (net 11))
 (segment (start 204.7834 58.039) (end 205.3168 57.1246) (width 0.19) (layer "B.Cu") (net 11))
 (segment (start 207.0186 54.1274) (end 207.0308 52.7952) (width 0.19) (layer "B.Cu") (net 11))
 (segment (start 194.471 61.5442) (end 197.2904 60.9112) (width 0.19) (layer "B.Cu") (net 11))
 (segment (start 204.123 58.3946) (end 204.7834 58.039) (width 0.19) (layer "B.Cu") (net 11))
 (segment (start 202.7768 58.8518) (end 204.123 58.3946) (width 0.19) (layer "B.Cu") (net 11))
 (segment (start 192.469 61.5086) (end 194.471 61.5442) (width 0.19) (layer "B.Cu") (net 11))
 (segment (start 204.5294 54.229) (end 204.4024 54.7878) (width 0.19) (layer "B.Cu") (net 11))
 (segment (start 199.3478 60.2996) (end 202.7768 58.8518) (width 0.19) (layer "B.Cu") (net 11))
 (segment (start 204.5308 52.7952) (end 204.5294 54.229) (width 0.19) (layer "B.Cu") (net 11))
 (segment (start 207.8568 55.245) (end 207.0186 54.1274) (width 0.19) (layer "B.Cu") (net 11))
 (segment (start 206.028 54.0766) (end 206.155 54.5846) (width 0.2) (layer "F.Cu") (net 20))
 (segment (start 206.0308 53.025201) (end 206.028 54.0766) (width 0.2) (layer "F.Cu") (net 20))
 (segment (start 206.536 55.2196) (end 206.6122 55.5752) (width 0.2) (layer "F.Cu") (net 20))
 (segment (start 206.6122 55.5752) (end 206.6376 55.8292) (width 0.2) (layer "F.Cu") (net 20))
 (segment (start 206.155 54.5846) (end 206.3836 55.0164) (width 0.2) (layer "F.Cu") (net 20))
 (segment (start 206.6376 55.8292) (end 206.0026 56.007) (width 0.2) (layer "F.Cu") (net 20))
 (segment (start 206.0026 56.007) (end 205.4438 55.9562) (width 0.2) (layer "F.Cu") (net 20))
 (segment (start 206.3836 55.0164) (end 206.536 55.2196) (width 0.2) (layer "F.Cu") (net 20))
 (via (at 206.6376 55.8292) (size 0.5) (drill 0.25) (layers "F.Cu" "B.Cu") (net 20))
 (via (at 205.4438 55.9562) (size 0.5) (drill 0.25) (layers "F.Cu" "B.Cu") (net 20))
 (segment (start 206.282 57.8612) (end 205.6216 59.0804) (width 0.2) (layer "B.Cu") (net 20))
 (segment (start 205.530801 53.0202) (end 205.5454 54.229) (width 0.2) (layer "B.Cu") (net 20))
 (segment (start 194 68.61) (end 194.01 67.8) (width 0.2) (layer "B.Cu") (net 20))
 (segment (start 198.3064 62.103) (end 195.995 63.2968) (width 0.2) (layer "B.Cu") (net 20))
 (segment (start 195.995 63.2968) (end 194.5472 64.6176) (width 0.2) (layer "B.Cu") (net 20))
 (segment (start 205.4438 55.9562) (end 205.393 55.4228) (width 0.2) (layer "B.Cu") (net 20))
 (segment (start 201.512656 61.076774) (end 198.3064 62.103) (width 0.2) (layer "B.Cu") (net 20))
 (segment (start 205.6216 59.0804) (end 204.4532 59.9948) (width 0.2) (layer "B.Cu") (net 20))
 (segment (start 204.4532 59.9948) (end 201.512656 61.076774) (width 0.2) (layer "B.Cu") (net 20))
 (segment (start 194.5472 64.6176) (end 194.1408 65.532) (width 0.2) (layer "B.Cu") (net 20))
 (segment (start 206.6376 55.8292) (end 206.282 57.8612) (width 0.2) (layer "B.Cu") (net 20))
 (segment (start 205.5454 54.229) (end 205.393 55.4228) (width 0.2) (layer "B.Cu") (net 20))
 (segment (start 194.1408 65.532) (end 194.01 67.8) (width 0.2) (layer "B.Cu") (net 20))
 (segment (start 205.9518 55.3974) (end 205.6216 54.737) (width 0.2) (layer "F.Cu") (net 17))
 (segment (start 205.5454 54.2036) (end 205.5308 53.025201) (width 0.2) (layer "F.Cu") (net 17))
 (segment (start 205.6216 54.737) (end 205.5454 54.2036) (width 0.2) (layer "F.Cu") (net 17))
 (via (at 205.9518 55.3974) (size 0.5) (drill 0.25) (layers "F.Cu" "B.Cu") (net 17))
 (segment (start 193.944953 64.8462) (end 194.1154 64.4144) (width 0.2) (layer "B.Cu") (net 17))
 (segment (start 194.5472 63.9826) (end 195.7664 62.9412) (width 0.2) (layer "B.Cu") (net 17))
 (segment (start 206.028 54.2544) (end 206.0788 54.864) (width 0.2) (layer "B.Cu") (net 17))
 (segment (start 195.7664 62.9412) (end 198.154 61.722) (width 0.2) (layer "B.Cu") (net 17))
 (segment (start 193.7344 65.3796) (end 193.944953 64.8462) (width 0.2) (layer "B.Cu") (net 17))
 (segment (start 205.9518 55.3974) (end 206.0788 55.5244) (width 0.2) (layer "B.Cu") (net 17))
 (segment (start 206.0308 53.020199) (end 206.028 54.2544) (width 0.2) (layer "B.Cu") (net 17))
 (segment (start 193.6 67.28) (end 193.7344 65.3796) (width 0.2) (layer "B.Cu") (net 17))
 (segment (start 194.1154 64.4144) (end 194.5472 63.9826) (width 0.2) (layer "B.Cu") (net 17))
 (segment (start 193.439473 64.9976) (end 193.944953 64.8462) (width 0.2) (layer "B.Cu") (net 17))
 (segment (start 193.6 68.61) (end 193.6 67.28) (width 0.2) (layer "B.Cu") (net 17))
 (segment (start 198.154 61.722) (end 201.456 60.6806) (width 0.2) (layer "B.Cu") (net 17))
 (segment (start 201.456 60.6806) (end 204.3516 59.563) (width 0.2) (layer "B.Cu") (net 17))
 (segment (start 206.0788 56.5658) (end 206.0788 55.5244) (width 0.2) (layer "B.Cu") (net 17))
 (segment (start 205.8756 57.658) (end 206.0788 56.5658) (width 0.2) (layer "B.Cu") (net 17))
 (segment (start 205.3422 58.7502) (end 205.8756 57.658) (width 0.2) (layer "B.Cu") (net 17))
 (segment (start 206.0788 54.864) (end 206.0788 55.5244) (width 0.2) (layer "B.Cu") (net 17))
 (segment (start 204.3516 59.563) (end 205.3422 58.7502) (width 0.2) (layer "B.Cu") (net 17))
 (segment (start 197.6206 72.0344) (end 198.2302 72.8218) (width 0.19) (layer "B.Cu") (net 13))
 (segment (start 195.7664 70.866) (end 196.249 71.0692) (width 0.19) (layer "B.Cu") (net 13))
 (segment (start 196.8078 71.4756) (end 197.6206 72.0344) (width 0.19) (layer "B.Cu") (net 13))
 (segment (start 195.05 70.86) (end 195.7664 70.866) (width 0.19) (layer "B.Cu") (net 13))
 (segment (start 196.249 71.0692) (end 196.8078 71.4756) (width 0.19) (layer "B.Cu") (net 13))
 (segment (start 193.0994 66.3448) (end 193.201 67.31) (width 0.19) (layer "B.Cu") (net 16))
 (segment (start 192.683127 65.5076) (end 193.0994 66.3448) (width 0.19) (layer "B.Cu") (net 16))
 (segment (start 193.201 67.31) (end 193.2 68.61) (width 0.19) (layer "B.Cu") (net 16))
 (via (at 133.8326 81.8896) (size 0.5) (drill 0.25) (layers "F.Cu" "B.Cu") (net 3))
 (segment (start 190.16 70.5) (end 133.8326 81.8896) (width 0.19) (layer "B.Cu") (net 3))
 (segment (start 192.15 70.46) (end 190.16 70.5) (width 0.19) (layer "B.Cu") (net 3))
 (via (at 138.7856 76.9888) (size 0.5) (drill 0.25) (layers "F.Cu" "B.Cu") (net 2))
 (segment (start 192.15 70.06) (end 190.21 70.1) (width 0.19) (layer "B.Cu") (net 2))
 (segment (start 190.21 70.1) (end 138.7856 76.9888) (width 0.19) (layer "B.Cu") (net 2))
 (via (at 220.2942 87.9094) (size 0.5) (drill 0.25) (layers "F.Cu" "B.Cu") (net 8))
 (segment (start 204.035 67.875) (end 220.2942 87.9094) (width 0.19) (layer "B.Cu") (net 8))
 (segment (start 195.76 69.251269) (end 197.86 68.325) (width 0.19) (layer "B.Cu") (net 8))
 (segment (start 203.51 67.35) (end 204.035 67.875) (width 0.19) (layer "B.Cu") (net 8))
 (segment (start 202.56 67.2) (end 203.51 67.35) (width 0.19) (layer "B.Cu") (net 8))
 (segment (start 195.05 69.26) (end 195.76 69.251269) (width 0.19) (layer "B.Cu") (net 8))
 (segment (start 197.86 68.325) (end 202.56 67.2) (width 0.19) (layer "B.Cu") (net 8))
 (via (at 204.1906 87.884) (size 0.5) (drill 0.25) (layers "F.Cu" "B.Cu") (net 1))
 (segment (start 194.4 71.51) (end 194.41 73.45) (width 0.19) (layer "B.Cu") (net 1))
 (segment (start 194.41 73.45) (end 204.1906 87.884) (width 0.19) (layer "B.Cu") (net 1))
 (via (at 182.4736 88.0364) (size 0.5) (drill 0.25) (layers "F.Cu" "B.Cu") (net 4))
 (segment (start 194 71.51) (end 194.01 73.9) (width 0.19) (layer "B.Cu") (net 4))
 (segment (start 194.01 73.9) (end 182.4736 88.0364) (width 0.19) (layer "B.Cu") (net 4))
 (via (at 166.4208 88.0872) (size 0.5) (drill 0.25) (layers "F.Cu" "B.Cu") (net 6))
 (segment (start 193.6 71.51) (end 193.61 73.45) (width 0.19) (layer "B.Cu") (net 6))
 (segment (start 193.61 73.45) (end 166.4208 88.0872) (width 0.19) (layer "B.Cu") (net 6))
 (via (at 138.7856 86.9682) (size 0.5) (drill 0.25) (layers "F.Cu" "B.Cu") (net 7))
 (segment (start 193.2 71.51) (end 193.21 72.65) (width 0.19) (layer "B.Cu") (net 7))
 (segment (start 193.21 72.65) (end 138.7856 86.9682) (width 0.19) (layer "B.Cu") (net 7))
 (via (at 143.8148 81.915) (size 0.5) (drill 0.25) (layers "F.Cu" "B.Cu") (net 5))
 (segment (start 192.81 72.15) (end 143.8148 81.915) (width 0.19) (layer "B.Cu") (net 5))
 (segment (start 192.8 71.51) (end 192.81 72.15) (width 0.19) (layer "B.Cu") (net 5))
 (segment (start 205.0374 54.0258) (end 205.0374 54.8132) (width 0.19) (layer "B.Cu") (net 15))
 (segment (start 204.9104 55.3974) (end 204.2266 57.2516) (width 0.19) (layer "B.Cu") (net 15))
 (segment (start 205.0308 53.0202) (end 205.0374 54.0258) (width 0.19) (layer "B.Cu") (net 15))
 (segment (start 205.0374 54.8132) (end 204.9104 55.3974) (width 0.19) (layer "B.Cu") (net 15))
 (segment (start 206.536 54.2798) (end 206.5308 53.0252) (width 0.19) (layer "F.Cu") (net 12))
 (segment (start 207.1456 55.2704) (end 206.536 54.2798) (width 0.19) (layer "F.Cu") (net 12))
 (via (at 207.1456 55.2704) (size 0.5) (drill 0.25) (layers "F.Cu" "B.Cu") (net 12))
 (segment (start 207.1456 55.2704) (end 207.2686 57.3024) (width 0.19) (layer "B.Cu") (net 12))
 (segment (start 198.8906 69.9262) (end 201.6084 69.8246) (width 0.19) (layer "B.Cu") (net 14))
 (segment (start 195.05 70.06) (end 196.11 70.05) (width 0.19) (layer "B.Cu") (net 14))
 (segment (start 196.11 70.05) (end 198.8906 69.9262) (width 0.19) (layer "B.Cu") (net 14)))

